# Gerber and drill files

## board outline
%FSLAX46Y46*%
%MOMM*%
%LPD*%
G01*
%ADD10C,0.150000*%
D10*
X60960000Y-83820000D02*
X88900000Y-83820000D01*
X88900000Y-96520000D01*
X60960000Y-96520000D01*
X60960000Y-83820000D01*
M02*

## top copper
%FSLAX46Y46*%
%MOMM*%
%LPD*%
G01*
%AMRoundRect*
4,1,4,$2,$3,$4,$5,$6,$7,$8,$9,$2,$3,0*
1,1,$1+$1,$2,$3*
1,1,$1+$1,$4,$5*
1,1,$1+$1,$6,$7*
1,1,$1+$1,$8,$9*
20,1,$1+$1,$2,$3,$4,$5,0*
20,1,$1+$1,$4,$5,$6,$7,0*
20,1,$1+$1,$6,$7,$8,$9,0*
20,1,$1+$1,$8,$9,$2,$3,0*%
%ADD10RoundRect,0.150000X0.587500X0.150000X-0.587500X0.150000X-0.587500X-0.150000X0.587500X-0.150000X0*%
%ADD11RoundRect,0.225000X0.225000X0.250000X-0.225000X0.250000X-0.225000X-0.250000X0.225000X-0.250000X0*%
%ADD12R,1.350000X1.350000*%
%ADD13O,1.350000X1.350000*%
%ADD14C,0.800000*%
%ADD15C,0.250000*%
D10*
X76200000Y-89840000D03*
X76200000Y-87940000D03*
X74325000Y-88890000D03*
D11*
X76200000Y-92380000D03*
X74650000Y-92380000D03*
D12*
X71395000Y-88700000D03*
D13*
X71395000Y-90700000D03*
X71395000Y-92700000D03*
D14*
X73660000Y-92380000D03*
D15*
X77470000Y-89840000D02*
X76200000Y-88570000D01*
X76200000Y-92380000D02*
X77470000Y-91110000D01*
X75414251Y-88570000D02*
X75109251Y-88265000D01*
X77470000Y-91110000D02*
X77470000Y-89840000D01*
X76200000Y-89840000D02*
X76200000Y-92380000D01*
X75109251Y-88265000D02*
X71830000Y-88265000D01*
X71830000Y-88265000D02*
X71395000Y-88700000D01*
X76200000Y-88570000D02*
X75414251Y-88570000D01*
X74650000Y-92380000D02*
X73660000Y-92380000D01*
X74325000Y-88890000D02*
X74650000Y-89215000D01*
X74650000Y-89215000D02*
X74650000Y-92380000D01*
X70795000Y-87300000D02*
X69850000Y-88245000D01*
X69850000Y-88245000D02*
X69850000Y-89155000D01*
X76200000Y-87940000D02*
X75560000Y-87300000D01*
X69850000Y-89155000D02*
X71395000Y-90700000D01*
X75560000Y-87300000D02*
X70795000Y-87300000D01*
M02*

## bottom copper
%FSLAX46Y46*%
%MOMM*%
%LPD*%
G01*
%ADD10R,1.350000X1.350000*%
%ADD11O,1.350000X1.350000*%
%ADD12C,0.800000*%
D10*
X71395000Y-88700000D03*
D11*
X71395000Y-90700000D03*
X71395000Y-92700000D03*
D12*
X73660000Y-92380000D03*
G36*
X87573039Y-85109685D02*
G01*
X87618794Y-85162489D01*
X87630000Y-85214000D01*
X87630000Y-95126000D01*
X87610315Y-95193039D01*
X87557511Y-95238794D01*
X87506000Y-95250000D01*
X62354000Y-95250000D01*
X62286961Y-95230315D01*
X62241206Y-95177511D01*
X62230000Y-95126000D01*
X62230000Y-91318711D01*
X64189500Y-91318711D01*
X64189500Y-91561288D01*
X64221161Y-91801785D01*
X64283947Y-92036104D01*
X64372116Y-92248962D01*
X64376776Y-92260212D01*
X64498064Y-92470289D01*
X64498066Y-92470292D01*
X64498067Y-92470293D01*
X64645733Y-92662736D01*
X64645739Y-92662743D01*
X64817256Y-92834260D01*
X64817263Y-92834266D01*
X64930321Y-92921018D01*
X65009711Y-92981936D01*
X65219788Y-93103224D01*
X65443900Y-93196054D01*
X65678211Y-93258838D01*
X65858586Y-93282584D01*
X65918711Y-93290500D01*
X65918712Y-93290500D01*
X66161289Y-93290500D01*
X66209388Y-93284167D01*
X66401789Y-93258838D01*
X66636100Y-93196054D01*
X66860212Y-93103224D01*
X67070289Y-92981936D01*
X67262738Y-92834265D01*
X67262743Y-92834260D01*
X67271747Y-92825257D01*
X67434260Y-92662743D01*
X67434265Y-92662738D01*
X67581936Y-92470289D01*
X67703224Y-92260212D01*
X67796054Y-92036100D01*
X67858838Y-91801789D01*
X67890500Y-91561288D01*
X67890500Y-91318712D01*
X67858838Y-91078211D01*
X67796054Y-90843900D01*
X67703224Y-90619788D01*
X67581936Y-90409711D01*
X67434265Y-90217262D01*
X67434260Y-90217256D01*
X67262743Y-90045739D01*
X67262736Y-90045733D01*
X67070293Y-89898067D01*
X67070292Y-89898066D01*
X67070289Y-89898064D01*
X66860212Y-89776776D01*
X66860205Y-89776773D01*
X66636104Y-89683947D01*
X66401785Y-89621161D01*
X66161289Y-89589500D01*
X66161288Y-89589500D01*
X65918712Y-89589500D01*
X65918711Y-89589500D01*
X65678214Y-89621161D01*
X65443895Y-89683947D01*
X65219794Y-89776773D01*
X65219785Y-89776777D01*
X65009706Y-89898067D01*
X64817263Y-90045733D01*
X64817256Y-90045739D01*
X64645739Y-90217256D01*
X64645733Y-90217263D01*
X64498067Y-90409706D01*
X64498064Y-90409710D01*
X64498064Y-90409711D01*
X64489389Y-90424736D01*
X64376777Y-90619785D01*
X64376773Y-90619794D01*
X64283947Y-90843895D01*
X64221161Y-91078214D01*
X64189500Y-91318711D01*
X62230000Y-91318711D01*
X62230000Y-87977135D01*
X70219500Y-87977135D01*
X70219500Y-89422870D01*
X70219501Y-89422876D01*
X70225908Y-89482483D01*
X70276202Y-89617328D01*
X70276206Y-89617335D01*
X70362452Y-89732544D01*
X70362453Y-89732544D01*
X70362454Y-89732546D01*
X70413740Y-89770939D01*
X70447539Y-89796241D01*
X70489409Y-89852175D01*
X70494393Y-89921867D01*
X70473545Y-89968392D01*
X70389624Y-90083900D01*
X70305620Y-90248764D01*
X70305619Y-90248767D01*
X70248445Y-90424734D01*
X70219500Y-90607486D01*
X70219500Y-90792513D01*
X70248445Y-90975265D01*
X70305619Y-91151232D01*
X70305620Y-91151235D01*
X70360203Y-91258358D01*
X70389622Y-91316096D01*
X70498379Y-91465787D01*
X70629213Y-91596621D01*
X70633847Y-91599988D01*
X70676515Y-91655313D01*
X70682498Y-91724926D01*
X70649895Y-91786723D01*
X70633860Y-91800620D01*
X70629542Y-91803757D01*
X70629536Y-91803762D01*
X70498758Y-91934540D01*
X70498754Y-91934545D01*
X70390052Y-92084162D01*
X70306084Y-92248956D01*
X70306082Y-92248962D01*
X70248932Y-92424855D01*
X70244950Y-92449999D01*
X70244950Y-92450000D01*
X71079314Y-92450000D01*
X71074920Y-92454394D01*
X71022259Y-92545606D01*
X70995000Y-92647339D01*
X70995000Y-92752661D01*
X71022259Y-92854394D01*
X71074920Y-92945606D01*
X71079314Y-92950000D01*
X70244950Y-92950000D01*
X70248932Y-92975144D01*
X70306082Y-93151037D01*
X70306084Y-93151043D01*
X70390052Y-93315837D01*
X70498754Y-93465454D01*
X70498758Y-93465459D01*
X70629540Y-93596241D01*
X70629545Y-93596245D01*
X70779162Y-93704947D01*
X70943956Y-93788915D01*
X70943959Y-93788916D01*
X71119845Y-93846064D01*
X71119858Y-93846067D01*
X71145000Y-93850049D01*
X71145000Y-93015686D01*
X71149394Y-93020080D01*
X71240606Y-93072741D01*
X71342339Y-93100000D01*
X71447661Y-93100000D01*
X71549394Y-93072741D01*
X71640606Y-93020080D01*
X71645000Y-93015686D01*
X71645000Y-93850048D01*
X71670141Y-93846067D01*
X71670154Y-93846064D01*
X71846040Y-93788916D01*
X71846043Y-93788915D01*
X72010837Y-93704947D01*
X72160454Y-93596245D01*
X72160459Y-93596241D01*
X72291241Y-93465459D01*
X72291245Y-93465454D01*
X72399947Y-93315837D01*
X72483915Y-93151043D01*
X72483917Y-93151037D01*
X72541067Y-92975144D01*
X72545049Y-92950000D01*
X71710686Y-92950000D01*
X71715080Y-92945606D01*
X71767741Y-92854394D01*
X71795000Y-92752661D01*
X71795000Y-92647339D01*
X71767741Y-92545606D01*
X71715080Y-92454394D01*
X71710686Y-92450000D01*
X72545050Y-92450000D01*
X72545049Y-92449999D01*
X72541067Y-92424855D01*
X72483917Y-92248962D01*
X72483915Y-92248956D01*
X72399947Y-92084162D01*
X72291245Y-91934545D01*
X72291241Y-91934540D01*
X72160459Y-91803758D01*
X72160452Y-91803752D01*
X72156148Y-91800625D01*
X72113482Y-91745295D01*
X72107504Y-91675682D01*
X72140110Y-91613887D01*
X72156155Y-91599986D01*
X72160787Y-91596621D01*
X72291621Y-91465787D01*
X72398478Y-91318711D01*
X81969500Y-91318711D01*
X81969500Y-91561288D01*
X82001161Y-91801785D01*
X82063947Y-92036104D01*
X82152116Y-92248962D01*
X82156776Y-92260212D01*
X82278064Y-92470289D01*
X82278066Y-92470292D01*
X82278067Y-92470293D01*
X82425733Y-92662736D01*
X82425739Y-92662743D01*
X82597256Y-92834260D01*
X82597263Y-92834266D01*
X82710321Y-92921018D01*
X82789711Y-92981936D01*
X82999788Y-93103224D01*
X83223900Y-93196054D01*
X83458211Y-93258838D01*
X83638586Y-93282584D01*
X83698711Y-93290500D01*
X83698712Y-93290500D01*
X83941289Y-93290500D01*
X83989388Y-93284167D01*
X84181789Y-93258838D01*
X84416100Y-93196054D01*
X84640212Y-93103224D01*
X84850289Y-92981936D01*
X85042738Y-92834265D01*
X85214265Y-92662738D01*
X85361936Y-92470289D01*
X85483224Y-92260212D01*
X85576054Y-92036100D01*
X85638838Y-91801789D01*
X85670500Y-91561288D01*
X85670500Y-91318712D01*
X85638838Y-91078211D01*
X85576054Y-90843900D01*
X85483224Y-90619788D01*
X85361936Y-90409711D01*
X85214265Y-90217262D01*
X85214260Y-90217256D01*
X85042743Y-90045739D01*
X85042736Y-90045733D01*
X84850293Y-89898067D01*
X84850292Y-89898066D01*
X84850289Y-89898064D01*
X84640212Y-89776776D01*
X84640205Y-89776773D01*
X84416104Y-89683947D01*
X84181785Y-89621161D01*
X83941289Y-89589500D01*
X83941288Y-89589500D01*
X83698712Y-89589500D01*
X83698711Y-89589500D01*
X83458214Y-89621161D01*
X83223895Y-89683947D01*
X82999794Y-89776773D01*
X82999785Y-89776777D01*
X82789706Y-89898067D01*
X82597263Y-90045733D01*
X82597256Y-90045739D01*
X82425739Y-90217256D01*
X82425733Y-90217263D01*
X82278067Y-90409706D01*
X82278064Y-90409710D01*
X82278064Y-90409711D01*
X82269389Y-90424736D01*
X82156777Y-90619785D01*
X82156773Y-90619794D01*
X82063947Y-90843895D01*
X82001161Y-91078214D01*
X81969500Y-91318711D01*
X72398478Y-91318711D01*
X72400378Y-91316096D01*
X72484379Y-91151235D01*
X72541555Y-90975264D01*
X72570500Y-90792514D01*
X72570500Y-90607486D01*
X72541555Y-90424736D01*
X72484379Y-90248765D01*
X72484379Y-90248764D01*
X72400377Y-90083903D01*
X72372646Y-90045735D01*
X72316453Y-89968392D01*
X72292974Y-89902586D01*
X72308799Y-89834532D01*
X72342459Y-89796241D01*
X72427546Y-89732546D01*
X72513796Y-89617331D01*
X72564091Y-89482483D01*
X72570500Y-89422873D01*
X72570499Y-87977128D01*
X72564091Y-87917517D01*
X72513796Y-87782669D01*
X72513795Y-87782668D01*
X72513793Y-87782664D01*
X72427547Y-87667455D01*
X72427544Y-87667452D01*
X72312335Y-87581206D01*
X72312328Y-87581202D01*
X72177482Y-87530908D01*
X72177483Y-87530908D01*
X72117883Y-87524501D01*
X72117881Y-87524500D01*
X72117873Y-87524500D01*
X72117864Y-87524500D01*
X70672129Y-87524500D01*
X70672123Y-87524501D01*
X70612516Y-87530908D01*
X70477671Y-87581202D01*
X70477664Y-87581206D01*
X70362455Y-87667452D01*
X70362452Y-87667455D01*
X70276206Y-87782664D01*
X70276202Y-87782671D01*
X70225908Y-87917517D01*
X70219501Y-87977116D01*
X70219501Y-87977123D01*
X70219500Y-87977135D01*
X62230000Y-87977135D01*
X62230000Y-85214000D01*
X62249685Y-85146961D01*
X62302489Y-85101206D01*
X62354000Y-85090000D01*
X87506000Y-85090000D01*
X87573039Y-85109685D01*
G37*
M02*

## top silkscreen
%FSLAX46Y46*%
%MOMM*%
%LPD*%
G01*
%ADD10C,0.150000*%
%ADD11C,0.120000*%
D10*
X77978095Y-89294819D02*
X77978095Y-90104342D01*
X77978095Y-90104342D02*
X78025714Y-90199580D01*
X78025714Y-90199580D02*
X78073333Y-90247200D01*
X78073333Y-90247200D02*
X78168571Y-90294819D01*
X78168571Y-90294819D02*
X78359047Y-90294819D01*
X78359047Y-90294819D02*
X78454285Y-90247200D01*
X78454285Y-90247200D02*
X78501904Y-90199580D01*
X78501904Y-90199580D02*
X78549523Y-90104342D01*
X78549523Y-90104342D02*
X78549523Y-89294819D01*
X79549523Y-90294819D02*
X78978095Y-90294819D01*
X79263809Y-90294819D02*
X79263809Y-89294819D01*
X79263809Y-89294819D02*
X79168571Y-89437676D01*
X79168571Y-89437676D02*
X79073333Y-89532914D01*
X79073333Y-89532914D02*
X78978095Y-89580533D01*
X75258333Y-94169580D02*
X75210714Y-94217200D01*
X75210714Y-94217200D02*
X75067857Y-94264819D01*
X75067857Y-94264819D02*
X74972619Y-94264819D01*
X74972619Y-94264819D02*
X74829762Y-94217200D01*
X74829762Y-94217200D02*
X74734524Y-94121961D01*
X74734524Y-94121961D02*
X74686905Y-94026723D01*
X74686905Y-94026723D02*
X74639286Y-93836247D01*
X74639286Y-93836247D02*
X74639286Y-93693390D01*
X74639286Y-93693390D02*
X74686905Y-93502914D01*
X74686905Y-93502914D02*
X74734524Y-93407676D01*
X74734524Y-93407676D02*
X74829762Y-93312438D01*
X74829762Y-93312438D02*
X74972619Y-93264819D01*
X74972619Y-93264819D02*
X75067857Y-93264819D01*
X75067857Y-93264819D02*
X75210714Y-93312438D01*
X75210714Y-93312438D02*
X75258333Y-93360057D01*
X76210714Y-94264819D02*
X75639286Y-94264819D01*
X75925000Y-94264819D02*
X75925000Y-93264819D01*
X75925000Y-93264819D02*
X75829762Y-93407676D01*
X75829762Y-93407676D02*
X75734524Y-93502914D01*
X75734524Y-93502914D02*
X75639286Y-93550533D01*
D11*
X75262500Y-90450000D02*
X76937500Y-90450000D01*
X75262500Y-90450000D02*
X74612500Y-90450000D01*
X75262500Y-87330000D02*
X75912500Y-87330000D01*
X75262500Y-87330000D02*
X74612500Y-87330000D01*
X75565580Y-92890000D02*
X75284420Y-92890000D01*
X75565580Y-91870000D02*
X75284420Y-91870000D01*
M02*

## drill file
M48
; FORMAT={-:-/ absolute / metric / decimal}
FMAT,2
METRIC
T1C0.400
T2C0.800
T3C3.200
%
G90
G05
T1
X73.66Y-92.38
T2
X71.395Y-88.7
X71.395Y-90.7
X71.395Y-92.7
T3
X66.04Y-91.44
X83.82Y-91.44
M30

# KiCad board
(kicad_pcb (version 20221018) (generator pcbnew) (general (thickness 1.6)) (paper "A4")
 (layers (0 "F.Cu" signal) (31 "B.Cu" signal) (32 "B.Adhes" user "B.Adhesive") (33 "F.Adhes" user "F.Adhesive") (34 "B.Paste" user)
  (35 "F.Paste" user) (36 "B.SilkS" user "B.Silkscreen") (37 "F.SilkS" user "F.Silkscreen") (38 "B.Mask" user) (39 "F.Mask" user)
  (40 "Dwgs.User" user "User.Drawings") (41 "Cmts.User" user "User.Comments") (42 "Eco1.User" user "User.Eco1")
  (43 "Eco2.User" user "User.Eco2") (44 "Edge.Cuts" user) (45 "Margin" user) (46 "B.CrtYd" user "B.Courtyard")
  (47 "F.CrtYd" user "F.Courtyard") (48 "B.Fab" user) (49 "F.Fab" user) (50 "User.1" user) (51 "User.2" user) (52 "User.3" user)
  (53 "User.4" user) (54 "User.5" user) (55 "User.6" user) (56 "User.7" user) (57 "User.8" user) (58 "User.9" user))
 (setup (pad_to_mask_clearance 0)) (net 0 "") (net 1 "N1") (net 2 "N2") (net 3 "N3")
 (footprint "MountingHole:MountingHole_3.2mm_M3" (layer "F.Cu") (at 83.82 91.44)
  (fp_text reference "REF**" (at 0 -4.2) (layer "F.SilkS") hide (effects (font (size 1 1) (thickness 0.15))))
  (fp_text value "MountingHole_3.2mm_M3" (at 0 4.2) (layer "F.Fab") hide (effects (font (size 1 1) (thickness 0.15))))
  (pad "" np_thru_hole circle (at 0 0) (size 3.2 3.2) (drill 3.2) (layers "*.Cu" "*.Mask")))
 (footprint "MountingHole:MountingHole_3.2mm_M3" (layer "F.Cu") (at 66.04 91.44)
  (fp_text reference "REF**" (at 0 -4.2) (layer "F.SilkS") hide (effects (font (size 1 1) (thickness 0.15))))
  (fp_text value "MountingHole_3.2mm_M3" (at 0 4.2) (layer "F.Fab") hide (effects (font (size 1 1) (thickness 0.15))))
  (pad "" np_thru_hole circle (at 0 0) (size 3.2 3.2) (drill 3.2) (layers "*.Cu" "*.Mask")))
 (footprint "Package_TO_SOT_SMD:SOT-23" (layer "F.Cu") (at 75.2625 88.89 180)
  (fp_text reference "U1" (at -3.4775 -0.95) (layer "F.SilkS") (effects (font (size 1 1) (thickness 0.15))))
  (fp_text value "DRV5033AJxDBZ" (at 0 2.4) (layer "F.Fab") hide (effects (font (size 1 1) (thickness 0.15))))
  (fp_line (start 0 -1.56) (end -1.675 -1.56) (stroke (width 0.12) (type solid)) (layer "F.SilkS"))
  (fp_line (start 0 -1.56) (end 0.65 -1.56) (stroke (width 0.12) (type solid)) (layer "F.SilkS"))
  (fp_line (start 0 1.56) (end -0.65 1.56) (stroke (width 0.12) (type solid)) (layer "F.SilkS"))
  (fp_line (start 0 1.56) (end 0.65 1.56) (stroke (width 0.12) (type solid)) (layer "F.SilkS"))
  (pad "1" smd roundrect (at -0.9375 -0.95 180) (size 1.475 0.6) (layers "F.Cu" "F.Paste" "F.Mask") (roundrect_rratio 0.25) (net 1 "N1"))
  (pad "2" smd roundrect (at -0.9375 0.95 180) (size 1.475 0.6) (layers "F.Cu" "F.Paste" "F.Mask") (roundrect_rratio 0.25) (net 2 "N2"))
  (pad "3" smd roundrect (at 0.9375 0 180) (size 1.475 0.6) (layers "F.Cu" "F.Paste" "F.Mask") (roundrect_rratio 0.25) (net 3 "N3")))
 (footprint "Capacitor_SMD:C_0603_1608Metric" (layer "F.Cu") (at 75.425 92.38 180)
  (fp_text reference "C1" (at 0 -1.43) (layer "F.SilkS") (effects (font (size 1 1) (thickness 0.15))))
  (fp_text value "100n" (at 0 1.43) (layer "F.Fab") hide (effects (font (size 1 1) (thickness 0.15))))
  (fp_line (start -0.14058 -0.51) (end 0.14058 -0.51) (stroke (width 0.12) (type solid)) (layer "F.SilkS"))
  (fp_line (start -0.14058 0.51) (end 0.14058 0.51) (stroke (width 0.12) (type solid)) (layer "F.SilkS"))
  (pad "1" smd roundrect (at -0.775 0 180) (size 0.9 0.95) (layers "F.Cu" "F.Paste" "F.Mask") (roundrect_rratio 0.25) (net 1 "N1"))
  (pad "2" smd roundrect (at 0.775 0 180) (size 0.9 0.95) (layers "F.Cu" "F.Paste" "F.Mask") (roundrect_rratio 0.25) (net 3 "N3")))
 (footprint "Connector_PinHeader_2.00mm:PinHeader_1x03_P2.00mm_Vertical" (layer "B.Cu") (at 71.395 88.7 180)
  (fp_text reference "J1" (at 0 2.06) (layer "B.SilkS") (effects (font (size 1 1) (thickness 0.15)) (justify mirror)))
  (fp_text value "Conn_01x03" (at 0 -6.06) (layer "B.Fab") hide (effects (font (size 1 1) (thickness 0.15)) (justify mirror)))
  (pad "1" thru_hole rect (at 0 0 180) (size 1.35 1.35) (drill 0.8) (layers "*.Cu" "*.Mask") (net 1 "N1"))
  (pad "2" thru_hole oval (at 0 -2 180) (size 1.35 1.35) (drill 0.8) (layers "*.Cu" "*.Mask") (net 2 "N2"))
  (pad "3" thru_hole oval (at 0 -4 180) (size 1.35 1.35) (drill 0.8) (layers "*.Cu" "*.Mask") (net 3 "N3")))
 (gr_rect (start 60.96 83.82) (end 88.9 96.52) (stroke (width 0.15) (type default)) (fill none) (layer "Edge.Cuts"))
 (segment (start 77.47 89.84) (end 76.2 88.57) (width 0.25) (layer "F.Cu") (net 1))
 (segment (start 76.2 92.38) (end 77.47 91.11) (width 0.25) (layer "F.Cu") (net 1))
 (segment (start 75.414251 88.57) (end 75.109251 88.265) (width 0.25) (layer "F.Cu") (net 1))
 (segment (start 77.47 91.11) (end 77.47 89.84) (width 0.25) (layer "F.Cu") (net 1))
 (segment (start 76.2 89.84) (end 76.2 92.38) (width 0.25) (layer "F.Cu") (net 1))
 (segment (start 75.109251 88.265) (end 71.83 88.265) (width 0.25) (layer "F.Cu") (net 1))
 (segment (start 71.83 88.265) (end 71.395 88.7) (width 0.25) (layer "F.Cu") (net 1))
 (segment (start 76.2 88.57) (end 75.414251 88.57) (width 0.25) (layer "F.Cu") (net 1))
 (segment (start 74.65 92.38) (end 73.66 92.38) (width 0.25) (layer "F.Cu") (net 3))
 (segment (start 74.325 88.89) (end 74.65 89.215) (width 0.25) (layer "F.Cu") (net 3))
 (segment (start 74.65 89.215) (end 74.65 92.38) (width 0.25) (layer "F.Cu") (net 3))
 (via (at 73.66 92.38) (size 0.8) (drill 0.4) (layers "F.Cu" "B.Cu") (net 3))
 (segment (start 70.795 87.3) (end 69.85 88.245) (width 0.25) (layer "F.Cu") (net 2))
 (segment (start 69.85 88.245) (end 69.85 89.155) (width 0.25) (layer "F.Cu") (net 2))
 (segment (start 76.2 87.94) (end 75.56 87.3) (width 0.25) (layer "F.Cu") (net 2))
 (segment (start 69.85 89.155) (end 71.395 90.7) (width 0.25) (layer "F.Cu") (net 2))
 (segment (start 75.56 87.3) (end 70.795 87.3) (width 0.25) (layer "F.Cu") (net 2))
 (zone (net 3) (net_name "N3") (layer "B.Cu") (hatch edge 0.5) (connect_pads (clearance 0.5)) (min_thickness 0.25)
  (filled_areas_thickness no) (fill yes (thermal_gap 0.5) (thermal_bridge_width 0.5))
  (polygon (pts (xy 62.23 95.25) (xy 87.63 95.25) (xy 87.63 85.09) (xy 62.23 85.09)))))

